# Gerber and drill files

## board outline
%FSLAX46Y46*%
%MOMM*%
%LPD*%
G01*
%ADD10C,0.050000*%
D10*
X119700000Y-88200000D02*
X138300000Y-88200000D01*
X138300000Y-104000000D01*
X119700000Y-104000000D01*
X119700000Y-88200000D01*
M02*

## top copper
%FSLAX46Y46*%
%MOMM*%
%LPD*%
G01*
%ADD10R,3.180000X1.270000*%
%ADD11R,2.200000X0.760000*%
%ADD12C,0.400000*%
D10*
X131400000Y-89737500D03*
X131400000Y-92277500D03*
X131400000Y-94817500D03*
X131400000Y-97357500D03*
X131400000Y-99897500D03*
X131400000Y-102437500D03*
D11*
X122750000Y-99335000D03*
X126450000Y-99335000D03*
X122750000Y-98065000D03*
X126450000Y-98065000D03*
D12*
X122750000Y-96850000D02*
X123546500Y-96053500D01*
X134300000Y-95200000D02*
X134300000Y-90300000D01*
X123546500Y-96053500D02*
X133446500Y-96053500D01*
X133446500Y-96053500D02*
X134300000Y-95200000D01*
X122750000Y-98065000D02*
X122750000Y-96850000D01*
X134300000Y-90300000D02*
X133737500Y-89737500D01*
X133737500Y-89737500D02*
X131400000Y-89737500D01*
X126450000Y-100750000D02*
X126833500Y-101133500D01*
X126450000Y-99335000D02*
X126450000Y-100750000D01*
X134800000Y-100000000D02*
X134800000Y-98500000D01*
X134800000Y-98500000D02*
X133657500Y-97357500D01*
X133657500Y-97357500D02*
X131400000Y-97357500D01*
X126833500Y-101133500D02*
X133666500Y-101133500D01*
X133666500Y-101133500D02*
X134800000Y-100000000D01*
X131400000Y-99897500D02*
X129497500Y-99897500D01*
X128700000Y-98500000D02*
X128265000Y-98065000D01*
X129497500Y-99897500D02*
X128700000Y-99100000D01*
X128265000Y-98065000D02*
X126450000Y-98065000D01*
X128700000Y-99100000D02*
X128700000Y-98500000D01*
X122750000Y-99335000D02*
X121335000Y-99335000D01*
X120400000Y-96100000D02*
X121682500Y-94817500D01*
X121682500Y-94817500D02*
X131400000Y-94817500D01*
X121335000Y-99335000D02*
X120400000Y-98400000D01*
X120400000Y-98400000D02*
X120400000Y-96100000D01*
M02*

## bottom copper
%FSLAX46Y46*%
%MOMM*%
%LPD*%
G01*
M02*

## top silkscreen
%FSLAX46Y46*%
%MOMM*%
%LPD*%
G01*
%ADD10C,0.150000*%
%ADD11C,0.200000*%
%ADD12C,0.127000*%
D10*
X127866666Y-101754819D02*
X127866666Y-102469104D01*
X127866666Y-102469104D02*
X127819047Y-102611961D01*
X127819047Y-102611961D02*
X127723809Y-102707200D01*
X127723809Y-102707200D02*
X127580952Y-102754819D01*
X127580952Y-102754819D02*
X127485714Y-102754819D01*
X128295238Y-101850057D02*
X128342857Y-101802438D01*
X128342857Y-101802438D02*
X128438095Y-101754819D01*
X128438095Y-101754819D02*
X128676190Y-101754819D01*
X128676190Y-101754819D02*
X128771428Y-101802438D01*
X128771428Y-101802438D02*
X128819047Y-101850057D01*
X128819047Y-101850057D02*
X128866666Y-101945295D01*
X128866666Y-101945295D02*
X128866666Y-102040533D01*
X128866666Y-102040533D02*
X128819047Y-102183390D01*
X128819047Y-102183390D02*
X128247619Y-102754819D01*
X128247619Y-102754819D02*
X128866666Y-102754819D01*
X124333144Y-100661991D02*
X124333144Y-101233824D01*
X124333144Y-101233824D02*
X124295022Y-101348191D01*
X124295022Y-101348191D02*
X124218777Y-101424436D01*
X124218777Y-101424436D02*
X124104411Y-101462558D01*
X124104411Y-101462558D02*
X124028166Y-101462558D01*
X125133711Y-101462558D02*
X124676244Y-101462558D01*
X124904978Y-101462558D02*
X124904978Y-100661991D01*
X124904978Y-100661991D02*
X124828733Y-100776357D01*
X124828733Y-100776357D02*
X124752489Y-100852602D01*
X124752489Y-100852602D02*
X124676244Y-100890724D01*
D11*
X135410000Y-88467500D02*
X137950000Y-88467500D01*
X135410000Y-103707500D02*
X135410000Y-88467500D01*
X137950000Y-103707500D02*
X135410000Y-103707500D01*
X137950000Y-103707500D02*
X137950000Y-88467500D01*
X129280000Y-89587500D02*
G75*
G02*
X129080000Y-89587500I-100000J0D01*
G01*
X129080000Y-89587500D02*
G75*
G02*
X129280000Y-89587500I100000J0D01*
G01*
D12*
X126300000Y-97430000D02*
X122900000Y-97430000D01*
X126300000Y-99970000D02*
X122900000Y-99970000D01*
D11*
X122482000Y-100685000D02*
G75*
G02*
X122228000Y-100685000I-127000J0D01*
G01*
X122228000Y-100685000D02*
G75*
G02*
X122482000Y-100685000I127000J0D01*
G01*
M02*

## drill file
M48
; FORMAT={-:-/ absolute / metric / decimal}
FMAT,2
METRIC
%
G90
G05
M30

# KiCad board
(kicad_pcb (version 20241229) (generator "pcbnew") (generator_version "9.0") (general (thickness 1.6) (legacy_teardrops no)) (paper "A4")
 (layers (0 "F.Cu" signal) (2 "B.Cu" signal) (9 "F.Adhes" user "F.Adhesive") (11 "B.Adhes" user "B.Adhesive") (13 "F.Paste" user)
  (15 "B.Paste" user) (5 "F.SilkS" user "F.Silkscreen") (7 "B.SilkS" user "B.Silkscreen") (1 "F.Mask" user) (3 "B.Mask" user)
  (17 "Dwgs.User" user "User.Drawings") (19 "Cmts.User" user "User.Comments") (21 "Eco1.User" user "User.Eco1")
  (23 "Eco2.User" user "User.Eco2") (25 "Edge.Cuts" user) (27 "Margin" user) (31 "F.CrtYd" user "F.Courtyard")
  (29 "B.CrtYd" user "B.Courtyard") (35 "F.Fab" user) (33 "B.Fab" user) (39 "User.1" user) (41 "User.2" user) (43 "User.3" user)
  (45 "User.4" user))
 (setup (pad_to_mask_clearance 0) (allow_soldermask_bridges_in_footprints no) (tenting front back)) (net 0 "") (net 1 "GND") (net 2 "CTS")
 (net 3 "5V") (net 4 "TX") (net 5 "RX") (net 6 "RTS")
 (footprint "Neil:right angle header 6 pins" (layer "F.Cu") (at 136.68 96.0875 -90)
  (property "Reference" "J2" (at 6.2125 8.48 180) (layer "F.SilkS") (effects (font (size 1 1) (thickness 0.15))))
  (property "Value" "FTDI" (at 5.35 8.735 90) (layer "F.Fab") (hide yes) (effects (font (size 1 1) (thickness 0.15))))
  (fp_line (start -7.62 1.27) (end -7.62 -1.27) (stroke (width 0.2) (type solid)) (layer "F.SilkS"))
  (fp_line (start 7.62 1.27) (end -7.62 1.27) (stroke (width 0.2) (type solid)) (layer "F.SilkS"))
  (fp_line (start 7.62 -1.27) (end 7.62 1.27) (stroke (width 0.2) (type solid)) (layer "F.SilkS"))
  (fp_line (start 7.62 -1.27) (end -7.62 -1.27) (stroke (width 0.2) (type solid)) (layer "F.SilkS"))
  (fp_circle (center -6.5 7.5) (end -6.4 7.5) (stroke (width 0.2) (type solid)) (fill no) (layer "F.SilkS"))
  (pad "01" smd rect (at -6.35 5.28 270) (size 1.27 3.18) (layers "F.Cu" "F.Mask" "F.Paste") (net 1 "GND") (solder_mask_margin 0.102))
  (pad "02" smd rect (at -3.81 5.28 270) (size 1.27 3.18) (layers "F.Cu" "F.Mask" "F.Paste") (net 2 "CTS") (solder_mask_margin 0.102))
  (pad "03" smd rect (at -1.27 5.28 270) (size 1.27 3.18) (layers "F.Cu" "F.Mask" "F.Paste") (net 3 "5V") (solder_mask_margin 0.102))
  (pad "04" smd rect (at 1.27 5.28 270) (size 1.27 3.18) (layers "F.Cu" "F.Mask" "F.Paste") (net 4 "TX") (solder_mask_margin 0.102))
  (pad "05" smd rect (at 3.81 5.28 270) (size 1.27 3.18) (layers "F.Cu" "F.Mask" "F.Paste") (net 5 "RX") (solder_mask_margin 0.102))
  (pad "06" smd rect (at 6.35 5.28 270) (size 1.27 3.18) (layers "F.Cu" "F.Mask" "F.Paste") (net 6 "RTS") (solder_mask_margin 0.102)))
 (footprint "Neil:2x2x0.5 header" (layer "F.Cu") (at 124.6 98.7 90)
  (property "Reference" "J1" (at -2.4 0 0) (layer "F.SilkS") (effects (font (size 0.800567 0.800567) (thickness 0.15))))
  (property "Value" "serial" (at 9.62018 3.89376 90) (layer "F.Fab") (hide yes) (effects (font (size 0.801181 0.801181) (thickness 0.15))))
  (fp_line (start 1.27 1.7) (end 1.27 -1.7) (stroke (width 0.127) (type solid)) (layer "F.SilkS"))
  (fp_line (start -1.27 1.7) (end -1.27 -1.7) (stroke (width 0.127) (type solid)) (layer "F.SilkS"))
  (fp_circle (center -1.985 -2.245) (end -1.858 -2.245) (stroke (width 0.2) (type solid)) (fill no) (layer "F.SilkS"))
  (pad "1" smd rect (at -0.635 -1.85 90) (size 0.76 2.2) (layers "F.Cu" "F.Mask" "F.Paste") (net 3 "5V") (solder_mask_margin 0.102))
  (pad "2" smd rect (at -0.635 1.85 90) (size 0.76 2.2) (layers "F.Cu" "F.Mask" "F.Paste") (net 4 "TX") (solder_mask_margin 0.102))
  (pad "3" smd rect (at 0.635 -1.85 90) (size 0.76 2.2) (layers "F.Cu" "F.Mask" "F.Paste") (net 1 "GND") (solder_mask_margin 0.102))
  (pad "4" smd rect (at 0.635 1.85 90) (size 0.76 2.2) (layers "F.Cu" "F.Mask" "F.Paste") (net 5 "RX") (solder_mask_margin 0.102)))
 (gr_rect (start 119.7 88.2) (end 138.3 104) (stroke (width 0.05) (type default)) (fill no) (layer "Edge.Cuts"))
 (segment (start 122.75 96.85) (end 123.5465 96.0535) (width 0.4) (layer "F.Cu") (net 1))
 (segment (start 134.3 95.2) (end 134.3 90.3) (width 0.4) (layer "F.Cu") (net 1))
 (segment (start 123.5465 96.0535) (end 133.4465 96.0535) (width 0.4) (layer "F.Cu") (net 1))
 (segment (start 133.4465 96.0535) (end 134.3 95.2) (width 0.4) (layer "F.Cu") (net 1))
 (segment (start 122.75 98.065) (end 122.75 96.85) (width 0.4) (layer "F.Cu") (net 1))
 (segment (start 134.3 90.3) (end 133.7375 89.7375) (width 0.4) (layer "F.Cu") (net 1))
 (segment (start 133.7375 89.7375) (end 131.4 89.7375) (width 0.4) (layer "F.Cu") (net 1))
 (segment (start 126.45 100.75) (end 126.8335 101.1335) (width 0.4) (layer "F.Cu") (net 4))
 (segment (start 126.45 99.335) (end 126.45 100.75) (width 0.4) (layer "F.Cu") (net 4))
 (segment (start 134.8 100) (end 134.8 98.5) (width 0.4) (layer "F.Cu") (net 4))
 (segment (start 134.8 98.5) (end 133.6575 97.3575) (width 0.4) (layer "F.Cu") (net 4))
 (segment (start 133.6575 97.3575) (end 131.4 97.3575) (width 0.4) (layer "F.Cu") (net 4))
 (segment (start 126.8335 101.1335) (end 133.6665 101.1335) (width 0.4) (layer "F.Cu") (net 4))
 (segment (start 133.6665 101.1335) (end 134.8 100) (width 0.4) (layer "F.Cu") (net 4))
 (segment (start 131.4 99.8975) (end 129.4975 99.8975) (width 0.4) (layer "F.Cu") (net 5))
 (segment (start 128.7 98.5) (end 128.265 98.065) (width 0.4) (layer "F.Cu") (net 5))
 (segment (start 129.4975 99.8975) (end 128.7 99.1) (width 0.4) (layer "F.Cu") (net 5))
 (segment (start 128.265 98.065) (end 126.45 98.065) (width 0.4) (layer "F.Cu") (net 5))
 (segment (start 128.7 99.1) (end 128.7 98.5) (width 0.4) (layer "F.Cu") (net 5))
 (segment (start 122.75 99.335) (end 121.335 99.335) (width 0.4) (layer "F.Cu") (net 3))
 (segment (start 120.4 96.1) (end 121.6825 94.8175) (width 0.4) (layer "F.Cu") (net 3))
 (segment (start 121.6825 94.8175) (end 131.4 94.8175) (width 0.4) (layer "F.Cu") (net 3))
 (segment (start 121.335 99.335) (end 120.4 98.4) (width 0.4) (layer "F.Cu") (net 3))
 (segment (start 120.4 98.4) (end 120.4 96.1) (width 0.4) (layer "F.Cu") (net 3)))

